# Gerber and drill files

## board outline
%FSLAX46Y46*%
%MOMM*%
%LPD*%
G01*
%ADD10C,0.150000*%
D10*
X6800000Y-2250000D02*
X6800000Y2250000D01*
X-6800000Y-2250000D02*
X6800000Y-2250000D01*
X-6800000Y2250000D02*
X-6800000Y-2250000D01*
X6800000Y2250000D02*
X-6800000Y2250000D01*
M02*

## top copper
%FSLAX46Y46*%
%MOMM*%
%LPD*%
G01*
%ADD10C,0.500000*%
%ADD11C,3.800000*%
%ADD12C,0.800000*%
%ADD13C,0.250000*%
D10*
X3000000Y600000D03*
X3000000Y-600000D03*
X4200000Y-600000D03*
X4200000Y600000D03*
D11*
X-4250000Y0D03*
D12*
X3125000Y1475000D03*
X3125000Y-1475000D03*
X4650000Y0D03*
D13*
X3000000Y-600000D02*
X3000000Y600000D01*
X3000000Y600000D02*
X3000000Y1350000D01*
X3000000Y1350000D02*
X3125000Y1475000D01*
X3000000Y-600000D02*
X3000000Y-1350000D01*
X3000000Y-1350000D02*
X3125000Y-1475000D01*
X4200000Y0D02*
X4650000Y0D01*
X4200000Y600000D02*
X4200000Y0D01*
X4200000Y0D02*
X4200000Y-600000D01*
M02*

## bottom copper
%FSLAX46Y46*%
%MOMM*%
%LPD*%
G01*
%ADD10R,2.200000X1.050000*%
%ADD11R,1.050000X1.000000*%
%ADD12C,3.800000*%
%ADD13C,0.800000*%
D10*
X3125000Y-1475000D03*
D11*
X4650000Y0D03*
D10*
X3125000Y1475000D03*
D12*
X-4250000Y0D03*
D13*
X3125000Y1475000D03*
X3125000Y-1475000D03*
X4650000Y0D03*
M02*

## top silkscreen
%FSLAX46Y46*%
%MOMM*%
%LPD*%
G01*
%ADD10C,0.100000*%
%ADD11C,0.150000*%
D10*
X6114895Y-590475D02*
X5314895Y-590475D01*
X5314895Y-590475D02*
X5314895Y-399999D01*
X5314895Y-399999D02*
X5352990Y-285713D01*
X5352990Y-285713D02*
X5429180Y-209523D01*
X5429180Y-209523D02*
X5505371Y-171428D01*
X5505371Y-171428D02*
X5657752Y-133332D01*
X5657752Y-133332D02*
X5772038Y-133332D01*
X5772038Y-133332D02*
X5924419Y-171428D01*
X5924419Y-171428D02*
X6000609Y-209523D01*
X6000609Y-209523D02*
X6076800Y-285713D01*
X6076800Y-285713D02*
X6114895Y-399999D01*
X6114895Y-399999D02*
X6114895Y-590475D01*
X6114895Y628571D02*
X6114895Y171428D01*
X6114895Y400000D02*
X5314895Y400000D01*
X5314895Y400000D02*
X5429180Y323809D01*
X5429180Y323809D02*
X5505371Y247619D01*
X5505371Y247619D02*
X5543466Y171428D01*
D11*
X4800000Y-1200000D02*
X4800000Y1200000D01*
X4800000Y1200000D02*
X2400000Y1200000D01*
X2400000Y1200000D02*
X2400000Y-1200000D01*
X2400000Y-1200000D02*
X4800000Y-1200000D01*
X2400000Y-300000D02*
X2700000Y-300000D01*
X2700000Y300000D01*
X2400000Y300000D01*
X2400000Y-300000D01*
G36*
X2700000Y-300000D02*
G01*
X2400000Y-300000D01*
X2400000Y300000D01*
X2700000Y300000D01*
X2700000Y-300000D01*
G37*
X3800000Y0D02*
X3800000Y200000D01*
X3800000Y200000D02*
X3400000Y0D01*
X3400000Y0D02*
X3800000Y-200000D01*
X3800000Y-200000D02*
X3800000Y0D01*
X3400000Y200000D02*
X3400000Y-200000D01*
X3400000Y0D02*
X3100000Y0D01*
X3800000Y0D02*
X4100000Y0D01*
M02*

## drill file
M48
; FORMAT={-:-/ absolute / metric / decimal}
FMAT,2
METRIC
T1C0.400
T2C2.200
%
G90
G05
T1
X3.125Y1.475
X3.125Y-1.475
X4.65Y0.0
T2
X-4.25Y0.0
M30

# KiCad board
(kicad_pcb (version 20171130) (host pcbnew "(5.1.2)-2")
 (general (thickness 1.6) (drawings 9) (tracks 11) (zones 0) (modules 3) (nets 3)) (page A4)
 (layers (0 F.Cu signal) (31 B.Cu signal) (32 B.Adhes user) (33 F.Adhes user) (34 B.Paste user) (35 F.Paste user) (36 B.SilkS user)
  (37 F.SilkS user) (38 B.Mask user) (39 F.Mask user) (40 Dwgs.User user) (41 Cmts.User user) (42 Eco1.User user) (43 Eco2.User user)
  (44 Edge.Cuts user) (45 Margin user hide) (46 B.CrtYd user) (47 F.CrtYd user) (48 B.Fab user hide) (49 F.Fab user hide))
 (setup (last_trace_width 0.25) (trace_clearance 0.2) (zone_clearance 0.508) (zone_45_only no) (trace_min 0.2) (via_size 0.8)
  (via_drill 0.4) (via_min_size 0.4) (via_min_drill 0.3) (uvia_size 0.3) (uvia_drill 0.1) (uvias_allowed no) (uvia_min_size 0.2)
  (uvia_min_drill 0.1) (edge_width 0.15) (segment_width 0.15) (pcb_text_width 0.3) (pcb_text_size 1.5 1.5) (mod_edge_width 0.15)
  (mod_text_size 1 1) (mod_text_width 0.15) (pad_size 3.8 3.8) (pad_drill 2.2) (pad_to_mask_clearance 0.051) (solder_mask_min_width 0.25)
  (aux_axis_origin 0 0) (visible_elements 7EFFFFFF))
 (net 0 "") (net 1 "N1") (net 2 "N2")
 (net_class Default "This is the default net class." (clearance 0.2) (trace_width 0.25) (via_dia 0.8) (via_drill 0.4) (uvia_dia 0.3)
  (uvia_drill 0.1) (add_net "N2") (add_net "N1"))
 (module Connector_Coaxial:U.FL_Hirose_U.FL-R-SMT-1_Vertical (layer B.Cu) (at 3.6 0 180)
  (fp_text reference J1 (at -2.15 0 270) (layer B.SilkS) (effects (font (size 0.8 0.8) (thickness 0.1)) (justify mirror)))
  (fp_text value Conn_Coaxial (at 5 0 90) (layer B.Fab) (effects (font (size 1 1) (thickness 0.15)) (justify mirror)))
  (pad 2 smd rect (at 0.475 -1.475 180) (size 2.2 1.05) (layers B.Cu B.Paste B.Mask) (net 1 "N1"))
  (pad 1 smd rect (at -1.05 0 180) (size 1.05 1) (layers B.Cu B.Paste B.Mask) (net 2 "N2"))
  (pad 2 smd rect (at 0.475 1.475 180) (size 2.2 1.05) (layers B.Cu B.Paste B.Mask) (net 1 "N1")))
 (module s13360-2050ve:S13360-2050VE (layer F.Cu) (at 3.6 0 270)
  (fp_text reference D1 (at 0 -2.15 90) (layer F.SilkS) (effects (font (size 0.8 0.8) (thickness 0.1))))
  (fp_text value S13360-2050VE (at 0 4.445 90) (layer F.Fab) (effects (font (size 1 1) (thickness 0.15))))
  (fp_line (start 1.2 -1.2) (end -1.2 -1.2) (layer F.SilkS) (width 0.15))
  (fp_line (start -1.2 -1.2) (end -1.2 1.2) (layer F.SilkS) (width 0.15))
  (fp_line (start -1.2 1.2) (end 1.2 1.2) (layer F.SilkS) (width 0.15))
  (fp_line (start 1.2 1.2) (end 1.2 -1.2) (layer F.SilkS) (width 0.15))
  (fp_poly (pts (xy 0.3 1.2) (xy 0.3 0.9) (xy -0.3 0.9) (xy -0.3 1.2)) (layer F.SilkS) (width 0.15))
  (fp_line (start 0 -0.2) (end -0.2 -0.2) (layer F.SilkS) (width 0.15))
  (fp_line (start -0.2 -0.2) (end 0 0.2) (layer F.SilkS) (width 0.15))
  (fp_line (start 0 0.2) (end 0.2 -0.2) (layer F.SilkS) (width 0.15))
  (fp_line (start 0.2 -0.2) (end 0 -0.2) (layer F.SilkS) (width 0.15))
  (fp_line (start -0.2 0.2) (end 0.2 0.2) (layer F.SilkS) (width 0.15))
  (fp_line (start 0 0.2) (end 0 0.5) (layer F.SilkS) (width 0.15))
  (fp_line (start 0 -0.2) (end 0 -0.5) (layer F.SilkS) (width 0.15))
  (pad 2 smd circle (at -0.6 0.6 270) (size 0.5 0.5) (layers F.Cu F.Paste F.Mask) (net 1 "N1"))
  (pad 2 smd circle (at 0.6 0.6 270) (size 0.5 0.5) (layers F.Cu F.Paste F.Mask) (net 1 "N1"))
  (pad 1 smd circle (at 0.6 -0.6 270) (size 0.5 0.5) (layers F.Cu F.Paste F.Mask) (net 2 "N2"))
  (pad 1 smd circle (at -0.6 -0.6 270) (size 0.5 0.5) (layers F.Cu F.Paste F.Mask) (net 2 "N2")))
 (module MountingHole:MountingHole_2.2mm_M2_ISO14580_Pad (layer F.Cu) (at -4.25 0)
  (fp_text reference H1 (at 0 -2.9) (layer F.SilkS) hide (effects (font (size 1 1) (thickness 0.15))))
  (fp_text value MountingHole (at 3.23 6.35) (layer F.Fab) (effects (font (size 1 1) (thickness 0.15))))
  (pad 1 thru_hole circle (at 0 0) (size 3.8 3.8) (drill 2.2) (layers *.Cu *.Mask)))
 (gr_line (start 6.8 2.25) (end 6.8 -2.25) (layer Edge.Cuts) (width 0.15))
 (gr_line (start -6.8 2.25) (end 6.8 2.25) (layer Edge.Cuts) (width 0.15))
 (gr_line (start -6.8 -2.25) (end -6.8 2.25) (layer Edge.Cuts) (width 0.15))
 (gr_line (start 6.8 -2.25) (end -6.8 -2.25) (layer Edge.Cuts) (width 0.15))
 (segment (start 3 0.6) (end 3 -0.6) (width 0.25) (layer F.Cu) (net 1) (status 30))
 (via (at 3.125 -1.475) (size 0.8) (drill 0.4) (layers F.Cu B.Cu) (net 1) (status 30))
 (segment (start 3 -0.6) (end 3 -1.35) (width 0.25) (layer F.Cu) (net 1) (status 10))
 (segment (start 3 -1.35) (end 3.125 -1.475) (width 0.25) (layer F.Cu) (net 1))
 (via (at 3.125 1.475) (size 0.8) (drill 0.4) (layers F.Cu B.Cu) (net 1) (status 30))
 (segment (start 3 0.6) (end 3 1.35) (width 0.25) (layer F.Cu) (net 1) (status 10))
 (segment (start 3 1.35) (end 3.125 1.475) (width 0.25) (layer F.Cu) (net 1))
 (via (at 4.65 0) (size 0.8) (drill 0.4) (layers F.Cu B.Cu) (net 2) (status 30))
 (segment (start 4.2 0) (end 4.65 0) (width 0.25) (layer F.Cu) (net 2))
 (segment (start 4.2 -0.6) (end 4.2 0) (width 0.25) (layer F.Cu) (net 2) (status 10))
 (segment (start 4.2 0) (end 4.2 0.6) (width 0.25) (layer F.Cu) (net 2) (status 20)))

